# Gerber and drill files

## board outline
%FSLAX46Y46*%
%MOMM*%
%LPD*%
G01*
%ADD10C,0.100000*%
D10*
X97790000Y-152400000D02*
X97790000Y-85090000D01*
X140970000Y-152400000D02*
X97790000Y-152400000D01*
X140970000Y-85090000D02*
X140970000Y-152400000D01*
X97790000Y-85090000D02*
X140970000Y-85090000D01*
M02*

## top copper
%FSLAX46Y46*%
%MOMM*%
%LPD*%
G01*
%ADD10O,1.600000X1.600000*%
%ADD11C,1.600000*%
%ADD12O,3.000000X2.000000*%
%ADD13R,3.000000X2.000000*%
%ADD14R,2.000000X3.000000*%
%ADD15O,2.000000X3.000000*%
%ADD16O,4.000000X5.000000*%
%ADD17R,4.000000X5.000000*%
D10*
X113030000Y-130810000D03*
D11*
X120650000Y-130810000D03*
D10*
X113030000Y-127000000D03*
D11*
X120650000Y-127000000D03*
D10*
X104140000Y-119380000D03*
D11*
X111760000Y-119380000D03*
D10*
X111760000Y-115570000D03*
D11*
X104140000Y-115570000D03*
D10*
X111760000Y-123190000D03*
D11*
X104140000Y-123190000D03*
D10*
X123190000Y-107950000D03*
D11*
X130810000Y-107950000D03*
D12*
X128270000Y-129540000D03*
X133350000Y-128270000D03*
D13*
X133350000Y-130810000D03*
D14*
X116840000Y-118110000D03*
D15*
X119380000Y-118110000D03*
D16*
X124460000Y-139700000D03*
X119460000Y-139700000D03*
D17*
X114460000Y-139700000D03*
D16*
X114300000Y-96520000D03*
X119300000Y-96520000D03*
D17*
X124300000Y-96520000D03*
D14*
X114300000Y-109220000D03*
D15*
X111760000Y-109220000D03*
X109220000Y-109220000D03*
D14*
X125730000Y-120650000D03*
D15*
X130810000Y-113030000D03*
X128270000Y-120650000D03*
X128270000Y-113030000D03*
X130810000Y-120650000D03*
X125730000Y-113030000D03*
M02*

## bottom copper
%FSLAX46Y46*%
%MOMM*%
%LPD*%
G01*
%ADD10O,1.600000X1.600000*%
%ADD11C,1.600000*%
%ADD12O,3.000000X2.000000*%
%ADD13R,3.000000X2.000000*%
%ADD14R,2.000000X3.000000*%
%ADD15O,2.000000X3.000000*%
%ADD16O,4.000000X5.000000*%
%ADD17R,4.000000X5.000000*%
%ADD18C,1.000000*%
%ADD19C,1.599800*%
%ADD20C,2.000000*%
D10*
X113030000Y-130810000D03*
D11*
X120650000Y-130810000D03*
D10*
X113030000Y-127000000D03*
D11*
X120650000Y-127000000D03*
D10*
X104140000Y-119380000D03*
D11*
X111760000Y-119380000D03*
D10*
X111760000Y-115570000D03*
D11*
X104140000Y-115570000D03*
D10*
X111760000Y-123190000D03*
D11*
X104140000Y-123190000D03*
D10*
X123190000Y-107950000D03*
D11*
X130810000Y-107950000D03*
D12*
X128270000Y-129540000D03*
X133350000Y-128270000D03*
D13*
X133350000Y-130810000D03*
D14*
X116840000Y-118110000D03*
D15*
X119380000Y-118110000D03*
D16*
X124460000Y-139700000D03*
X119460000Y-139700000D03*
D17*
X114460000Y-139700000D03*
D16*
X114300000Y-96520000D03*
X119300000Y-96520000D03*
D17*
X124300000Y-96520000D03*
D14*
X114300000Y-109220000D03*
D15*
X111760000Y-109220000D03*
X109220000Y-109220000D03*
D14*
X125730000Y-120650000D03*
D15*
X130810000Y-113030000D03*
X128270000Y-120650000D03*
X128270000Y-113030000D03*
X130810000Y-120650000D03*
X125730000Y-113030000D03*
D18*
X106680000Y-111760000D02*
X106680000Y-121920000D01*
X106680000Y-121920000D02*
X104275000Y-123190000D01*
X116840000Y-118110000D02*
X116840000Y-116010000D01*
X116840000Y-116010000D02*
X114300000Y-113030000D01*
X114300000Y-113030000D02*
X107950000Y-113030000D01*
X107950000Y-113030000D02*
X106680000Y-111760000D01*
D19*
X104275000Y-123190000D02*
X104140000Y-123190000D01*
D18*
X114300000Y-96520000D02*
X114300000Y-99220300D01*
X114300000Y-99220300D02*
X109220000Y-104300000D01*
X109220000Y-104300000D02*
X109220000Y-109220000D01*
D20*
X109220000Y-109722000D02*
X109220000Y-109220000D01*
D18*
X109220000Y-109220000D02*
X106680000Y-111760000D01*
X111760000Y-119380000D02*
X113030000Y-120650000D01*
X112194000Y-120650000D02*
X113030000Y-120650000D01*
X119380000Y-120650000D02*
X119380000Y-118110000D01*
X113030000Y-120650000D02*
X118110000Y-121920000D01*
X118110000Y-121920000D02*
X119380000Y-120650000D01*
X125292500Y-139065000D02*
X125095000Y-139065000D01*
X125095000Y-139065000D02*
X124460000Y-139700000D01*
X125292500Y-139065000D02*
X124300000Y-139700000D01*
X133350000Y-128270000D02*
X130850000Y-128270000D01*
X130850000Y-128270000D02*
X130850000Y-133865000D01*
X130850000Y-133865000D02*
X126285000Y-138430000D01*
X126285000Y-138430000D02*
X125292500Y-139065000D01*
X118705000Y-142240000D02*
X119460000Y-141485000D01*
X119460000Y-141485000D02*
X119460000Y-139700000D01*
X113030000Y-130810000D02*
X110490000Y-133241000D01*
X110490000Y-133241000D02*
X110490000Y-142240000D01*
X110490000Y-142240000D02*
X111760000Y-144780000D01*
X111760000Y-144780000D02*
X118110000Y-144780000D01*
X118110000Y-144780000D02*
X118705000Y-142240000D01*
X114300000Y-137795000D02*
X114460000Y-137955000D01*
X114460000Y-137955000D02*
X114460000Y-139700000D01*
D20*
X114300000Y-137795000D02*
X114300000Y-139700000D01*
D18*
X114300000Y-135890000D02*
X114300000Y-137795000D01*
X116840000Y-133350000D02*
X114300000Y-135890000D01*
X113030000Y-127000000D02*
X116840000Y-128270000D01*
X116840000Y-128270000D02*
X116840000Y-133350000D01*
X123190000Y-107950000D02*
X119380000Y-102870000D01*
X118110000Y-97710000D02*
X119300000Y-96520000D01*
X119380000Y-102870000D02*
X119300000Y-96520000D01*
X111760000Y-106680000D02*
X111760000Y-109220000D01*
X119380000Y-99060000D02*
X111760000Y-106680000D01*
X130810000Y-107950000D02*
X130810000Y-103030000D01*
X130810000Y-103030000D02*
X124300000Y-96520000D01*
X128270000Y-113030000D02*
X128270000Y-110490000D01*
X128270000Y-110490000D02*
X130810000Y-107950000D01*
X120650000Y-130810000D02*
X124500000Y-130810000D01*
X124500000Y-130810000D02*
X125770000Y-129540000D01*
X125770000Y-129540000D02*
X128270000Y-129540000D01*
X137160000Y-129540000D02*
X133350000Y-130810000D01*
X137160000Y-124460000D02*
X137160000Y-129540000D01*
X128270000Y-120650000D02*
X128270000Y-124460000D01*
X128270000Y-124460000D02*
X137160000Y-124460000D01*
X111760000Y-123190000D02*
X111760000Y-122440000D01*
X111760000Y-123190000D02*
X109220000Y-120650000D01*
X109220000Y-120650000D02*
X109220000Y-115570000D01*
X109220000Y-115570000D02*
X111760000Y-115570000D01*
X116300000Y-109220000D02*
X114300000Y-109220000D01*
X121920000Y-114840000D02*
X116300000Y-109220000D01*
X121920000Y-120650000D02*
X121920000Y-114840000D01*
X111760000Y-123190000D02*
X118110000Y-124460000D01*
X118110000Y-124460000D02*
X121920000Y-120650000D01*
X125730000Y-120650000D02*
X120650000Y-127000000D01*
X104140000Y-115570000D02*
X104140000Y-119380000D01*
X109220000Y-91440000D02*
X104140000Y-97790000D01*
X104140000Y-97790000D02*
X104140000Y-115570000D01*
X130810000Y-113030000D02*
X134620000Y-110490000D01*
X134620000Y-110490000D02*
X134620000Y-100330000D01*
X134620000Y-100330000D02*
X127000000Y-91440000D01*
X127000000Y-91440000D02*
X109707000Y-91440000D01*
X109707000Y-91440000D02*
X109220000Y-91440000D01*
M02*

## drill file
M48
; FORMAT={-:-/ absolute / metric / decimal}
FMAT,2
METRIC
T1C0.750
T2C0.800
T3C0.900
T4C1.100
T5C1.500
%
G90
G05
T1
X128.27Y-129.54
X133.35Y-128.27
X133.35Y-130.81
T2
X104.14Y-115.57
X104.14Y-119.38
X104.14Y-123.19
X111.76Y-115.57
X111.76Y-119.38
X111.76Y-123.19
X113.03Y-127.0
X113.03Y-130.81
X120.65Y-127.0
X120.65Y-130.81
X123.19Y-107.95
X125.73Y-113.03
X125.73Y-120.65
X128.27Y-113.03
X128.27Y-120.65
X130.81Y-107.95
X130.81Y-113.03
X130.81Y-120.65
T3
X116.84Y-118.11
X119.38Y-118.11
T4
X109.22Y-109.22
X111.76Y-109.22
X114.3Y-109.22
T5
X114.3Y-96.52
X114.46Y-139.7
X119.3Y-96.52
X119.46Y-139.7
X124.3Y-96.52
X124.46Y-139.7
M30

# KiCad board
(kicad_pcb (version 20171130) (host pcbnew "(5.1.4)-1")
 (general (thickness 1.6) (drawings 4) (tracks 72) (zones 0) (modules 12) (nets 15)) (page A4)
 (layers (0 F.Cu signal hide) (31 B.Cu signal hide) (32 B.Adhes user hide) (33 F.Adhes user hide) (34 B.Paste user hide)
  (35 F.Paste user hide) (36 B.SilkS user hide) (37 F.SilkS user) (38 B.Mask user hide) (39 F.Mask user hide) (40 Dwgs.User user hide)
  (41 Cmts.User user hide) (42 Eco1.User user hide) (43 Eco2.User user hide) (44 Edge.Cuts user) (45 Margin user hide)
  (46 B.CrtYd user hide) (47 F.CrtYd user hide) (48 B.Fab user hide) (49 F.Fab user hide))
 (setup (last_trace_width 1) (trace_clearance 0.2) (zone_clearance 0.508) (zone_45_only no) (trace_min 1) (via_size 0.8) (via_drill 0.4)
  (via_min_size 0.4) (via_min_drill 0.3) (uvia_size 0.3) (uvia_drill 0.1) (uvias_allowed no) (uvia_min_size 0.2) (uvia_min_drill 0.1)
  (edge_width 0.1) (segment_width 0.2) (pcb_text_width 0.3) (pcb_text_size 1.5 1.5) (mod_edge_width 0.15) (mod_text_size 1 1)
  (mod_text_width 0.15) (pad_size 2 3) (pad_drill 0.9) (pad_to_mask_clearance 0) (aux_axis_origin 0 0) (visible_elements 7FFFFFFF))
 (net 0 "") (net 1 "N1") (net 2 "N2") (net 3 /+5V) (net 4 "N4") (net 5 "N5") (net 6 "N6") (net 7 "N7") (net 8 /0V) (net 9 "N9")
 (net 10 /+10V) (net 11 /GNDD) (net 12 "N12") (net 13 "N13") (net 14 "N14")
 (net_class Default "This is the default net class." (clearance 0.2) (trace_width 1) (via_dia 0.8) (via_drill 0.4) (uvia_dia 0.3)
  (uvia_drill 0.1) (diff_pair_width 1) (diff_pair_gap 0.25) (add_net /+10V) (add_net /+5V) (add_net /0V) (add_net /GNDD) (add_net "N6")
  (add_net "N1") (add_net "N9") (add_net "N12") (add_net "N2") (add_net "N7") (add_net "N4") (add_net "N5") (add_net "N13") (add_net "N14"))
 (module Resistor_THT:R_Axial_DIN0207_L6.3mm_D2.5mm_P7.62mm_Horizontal (layer F.Cu) (at 120.65 130.81 180)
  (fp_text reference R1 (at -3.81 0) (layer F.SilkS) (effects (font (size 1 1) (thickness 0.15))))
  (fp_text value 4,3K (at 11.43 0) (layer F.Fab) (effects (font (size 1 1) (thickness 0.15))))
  (pad 2 thru_hole oval (at 7.62 0 180) (size 1.6 1.6) (drill 0.8) (layers *.Cu *.Mask) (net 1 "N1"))
  (pad 1 thru_hole circle (at 0 0 180) (size 1.6 1.6) (drill 0.8) (layers *.Cu *.Mask) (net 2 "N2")))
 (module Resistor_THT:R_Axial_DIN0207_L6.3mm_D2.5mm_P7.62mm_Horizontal (layer F.Cu) (at 120.65 127 180)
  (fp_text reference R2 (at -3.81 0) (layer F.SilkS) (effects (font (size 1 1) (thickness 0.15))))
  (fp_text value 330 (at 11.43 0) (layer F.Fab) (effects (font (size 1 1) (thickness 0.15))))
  (pad 2 thru_hole oval (at 7.62 0 180) (size 1.6 1.6) (drill 0.8) (layers *.Cu *.Mask) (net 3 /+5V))
  (pad 1 thru_hole circle (at 0 0 180) (size 1.6 1.6) (drill 0.8) (layers *.Cu *.Mask) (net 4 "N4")))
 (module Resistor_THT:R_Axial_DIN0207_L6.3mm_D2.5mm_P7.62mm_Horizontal (layer F.Cu) (at 111.76 119.38 180)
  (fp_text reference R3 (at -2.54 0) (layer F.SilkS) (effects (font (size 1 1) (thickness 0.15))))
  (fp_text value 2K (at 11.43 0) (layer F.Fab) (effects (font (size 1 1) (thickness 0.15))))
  (pad 2 thru_hole oval (at 7.62 0 180) (size 1.6 1.6) (drill 0.8) (layers *.Cu *.Mask) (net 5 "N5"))
  (pad 1 thru_hole circle (at 0 0 180) (size 1.6 1.6) (drill 0.8) (layers *.Cu *.Mask) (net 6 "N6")))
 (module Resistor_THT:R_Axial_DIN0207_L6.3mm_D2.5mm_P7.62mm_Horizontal (layer F.Cu) (at 104.14 115.57)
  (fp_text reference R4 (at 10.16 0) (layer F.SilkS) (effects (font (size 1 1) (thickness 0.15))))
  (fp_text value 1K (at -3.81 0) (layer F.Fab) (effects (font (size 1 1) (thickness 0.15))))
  (pad 2 thru_hole oval (at 7.62 0) (size 1.6 1.6) (drill 0.8) (layers *.Cu *.Mask) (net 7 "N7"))
  (pad 1 thru_hole circle (at 0 0) (size 1.6 1.6) (drill 0.8) (layers *.Cu *.Mask) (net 5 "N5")))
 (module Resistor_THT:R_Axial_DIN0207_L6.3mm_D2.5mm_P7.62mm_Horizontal (layer F.Cu) (at 104.14 123.19)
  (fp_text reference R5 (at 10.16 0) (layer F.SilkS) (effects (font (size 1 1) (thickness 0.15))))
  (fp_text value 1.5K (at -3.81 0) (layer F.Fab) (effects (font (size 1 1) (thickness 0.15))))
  (pad 2 thru_hole oval (at 7.62 0) (size 1.6 1.6) (drill 0.8) (layers *.Cu *.Mask) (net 7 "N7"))
  (pad 1 thru_hole circle (at 0 0) (size 1.6 1.6) (drill 0.8) (layers *.Cu *.Mask) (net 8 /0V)))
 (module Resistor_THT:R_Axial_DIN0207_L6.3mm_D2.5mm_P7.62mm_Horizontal (layer F.Cu) (at 130.81 107.95 180)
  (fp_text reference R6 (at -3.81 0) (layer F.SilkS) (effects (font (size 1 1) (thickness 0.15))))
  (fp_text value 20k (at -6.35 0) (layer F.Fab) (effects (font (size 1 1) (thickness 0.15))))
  (pad 2 thru_hole oval (at 7.62 0 180) (size 1.6 1.6) (drill 0.8) (layers *.Cu *.Mask) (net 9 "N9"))
  (pad 1 thru_hole circle (at 0 0 180) (size 1.6 1.6) (drill 0.8) (layers *.Cu *.Mask) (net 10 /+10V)))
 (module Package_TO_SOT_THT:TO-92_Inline (layer F.Cu) (at 133.35 130.81 90)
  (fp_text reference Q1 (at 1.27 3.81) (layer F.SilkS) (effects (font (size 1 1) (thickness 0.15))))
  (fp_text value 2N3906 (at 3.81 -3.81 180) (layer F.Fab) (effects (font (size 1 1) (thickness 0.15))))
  (pad 2 thru_hole oval (at 1.27 -5.08 90) (size 2 3) (drill 0.75) (layers *.Cu *.Mask) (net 2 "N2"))
  (pad 3 thru_hole oval (at 2.54 0 90) (size 2 3) (drill 0.75) (layers *.Cu *.Mask) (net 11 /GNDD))
  (pad 1 thru_hole rect (at 0 0 90) (size 2 3) (drill 0.75) (layers *.Cu *.Mask) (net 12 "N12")))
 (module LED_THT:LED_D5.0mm (layer F.Cu) (at 116.84 118.11)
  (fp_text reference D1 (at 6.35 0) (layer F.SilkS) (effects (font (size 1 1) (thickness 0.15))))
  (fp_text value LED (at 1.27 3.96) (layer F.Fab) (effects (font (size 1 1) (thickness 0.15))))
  (pad 1 thru_hole rect (at 0 0) (size 2 3) (drill 0.9) (layers *.Cu *.Mask) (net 8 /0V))
  (pad 2 thru_hole oval (at 2.54 0) (size 2 3) (drill 0.9) (layers *.Cu *.Mask) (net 6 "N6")))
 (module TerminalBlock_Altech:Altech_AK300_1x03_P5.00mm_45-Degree (layer F.Cu) (at 114.46 139.7)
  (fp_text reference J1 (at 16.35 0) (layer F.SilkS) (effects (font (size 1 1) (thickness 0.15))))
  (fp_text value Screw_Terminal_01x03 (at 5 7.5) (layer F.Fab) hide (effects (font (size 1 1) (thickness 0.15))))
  (pad 3 thru_hole oval (at 10 0) (size 4 5) (drill 1.5) (layers *.Cu *.Mask) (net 11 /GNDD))
  (pad 2 thru_hole oval (at 5 0) (size 4 5) (drill 1.5) (layers *.Cu *.Mask) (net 1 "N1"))
  (pad 1 thru_hole rect (at 0 0) (size 4 5) (drill 1.5) (layers *.Cu *.Mask) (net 3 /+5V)))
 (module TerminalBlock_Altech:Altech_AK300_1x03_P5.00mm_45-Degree (layer F.Cu) (at 114.3 96.52)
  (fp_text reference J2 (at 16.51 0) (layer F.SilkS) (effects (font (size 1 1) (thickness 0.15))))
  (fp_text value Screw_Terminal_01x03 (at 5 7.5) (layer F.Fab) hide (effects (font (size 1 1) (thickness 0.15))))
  (pad 1 thru_hole oval (at 0 0) (size 4 5) (drill 1.5) (layers *.Cu *.Mask) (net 8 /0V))
  (pad 2 thru_hole oval (at 5 0) (size 4 5) (drill 1.5) (layers *.Cu *.Mask) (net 9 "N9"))
  (pad 3 thru_hole rect (at 10 0) (size 4 5) (drill 1.5) (layers *.Cu *.Mask) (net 10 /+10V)))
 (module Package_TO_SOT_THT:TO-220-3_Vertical (layer F.Cu) (at 114.3 109.22 180)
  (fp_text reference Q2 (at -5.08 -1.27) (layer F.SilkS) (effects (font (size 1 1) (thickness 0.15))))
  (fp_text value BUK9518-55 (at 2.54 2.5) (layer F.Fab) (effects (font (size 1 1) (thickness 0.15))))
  (pad 1 thru_hole rect (at 0 0 180) (size 2 3) (drill 1.1) (layers *.Cu *.Mask) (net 7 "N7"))
  (pad 2 thru_hole oval (at 2.54 0 180) (size 2 3) (drill 1.1) (layers *.Cu *.Mask) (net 9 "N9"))
  (pad 3 thru_hole oval (at 5.08 0 180) (size 2 3) (drill 1.1) (layers *.Cu *.Mask) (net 8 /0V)))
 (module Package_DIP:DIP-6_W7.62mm (layer F.Cu) (at 125.73 120.65 90)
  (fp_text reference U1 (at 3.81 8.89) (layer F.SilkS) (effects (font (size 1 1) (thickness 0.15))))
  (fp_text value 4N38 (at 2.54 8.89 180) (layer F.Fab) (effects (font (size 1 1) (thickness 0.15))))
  (pad 1 thru_hole rect (at 0 0 90) (size 3 2) (drill 0.8) (layers *.Cu *.Mask) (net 4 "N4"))
  (pad 4 thru_hole oval (at 7.62 5.08 90) (size 3 2) (drill 0.8) (layers *.Cu *.Mask) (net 5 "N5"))
  (pad 2 thru_hole oval (at 0 2.54 90) (size 3 2) (drill 0.8) (layers *.Cu *.Mask) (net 12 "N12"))
  (pad 5 thru_hole oval (at 7.62 2.54 90) (size 3 2) (drill 0.8) (layers *.Cu *.Mask) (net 10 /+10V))
  (pad 3 thru_hole oval (at 0 5.08 90) (size 3 2) (drill 0.8) (layers *.Cu *.Mask) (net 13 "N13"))
  (pad 6 thru_hole oval (at 7.62 0 90) (size 3 2) (drill 0.8) (layers *.Cu *.Mask) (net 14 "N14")))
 (gr_line (start 97.79 152.4) (end 97.79 85.09) (layer Edge.Cuts) (width 0.1))
 (gr_line (start 140.97 152.4) (end 97.79 152.4) (layer Edge.Cuts) (width 0.1))
 (gr_line (start 140.97 85.09) (end 140.97 152.4) (layer Edge.Cuts) (width 0.1))
 (gr_line (start 97.79 85.09) (end 140.97 85.09) (layer Edge.Cuts) (width 0.1))
 (segment (start 106.68 111.76) (end 106.68 121.92) (width 1) (layer B.Cu) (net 8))
 (segment (start 106.68 121.92) (end 104.275 123.19) (width 1) (layer B.Cu) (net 8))
 (segment (start 116.84 118.11) (end 116.84 116.01) (width 1) (layer B.Cu) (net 8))
 (segment (start 116.84 116.01) (end 114.3 113.03) (width 1) (layer B.Cu) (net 8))
 (segment (start 114.3 113.03) (end 107.95 113.03) (width 1) (layer B.Cu) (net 8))
 (segment (start 107.95 113.03) (end 106.68 111.76) (width 1) (layer B.Cu) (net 8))
 (segment (start 104.275 123.19) (end 104.14 123.19) (width 1.5998) (layer B.Cu) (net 8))
 (segment (start 114.3 96.52) (end 114.3 99.2203) (width 1) (layer B.Cu) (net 8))
 (segment (start 114.3 99.2203) (end 109.22 104.3) (width 1) (layer B.Cu) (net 8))
 (segment (start 109.22 104.3) (end 109.22 109.22) (width 1) (layer B.Cu) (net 8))
 (segment (start 109.22 109.722) (end 109.22 109.22) (width 2) (layer B.Cu) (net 8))
 (segment (start 109.22 109.22) (end 106.68 111.76) (width 1) (layer B.Cu) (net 8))
 (segment (start 111.76 119.38) (end 113.03 120.65) (width 1) (layer B.Cu) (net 6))
 (segment (start 112.194 120.65) (end 113.03 120.65) (width 1) (layer B.Cu) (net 6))
 (segment (start 119.38 120.65) (end 119.38 118.11) (width 1) (layer B.Cu) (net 6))
 (segment (start 113.03 120.65) (end 118.11 121.92) (width 1) (layer B.Cu) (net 6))
 (segment (start 118.11 121.92) (end 119.38 120.65) (width 1) (layer B.Cu) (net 6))
 (segment (start 125.2925 139.065) (end 125.095 139.065) (width 1) (layer B.Cu) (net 11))
 (segment (start 125.095 139.065) (end 124.46 139.7) (width 1) (layer B.Cu) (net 11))
 (segment (start 125.2925 139.065) (end 124.3 139.7) (width 1) (layer B.Cu) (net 11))
 (segment (start 133.35 128.27) (end 130.85 128.27) (width 1) (layer B.Cu) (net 11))
 (segment (start 130.85 128.27) (end 130.85 133.865) (width 1) (layer B.Cu) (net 11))
 (segment (start 130.85 133.865) (end 126.285 138.43) (width 1) (layer B.Cu) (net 11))
 (segment (start 126.285 138.43) (end 125.2925 139.065) (width 1) (layer B.Cu) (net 11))
 (segment (start 118.705 142.24) (end 119.46 141.485) (width 1) (layer B.Cu) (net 1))
 (segment (start 119.46 141.485) (end 119.46 139.7) (width 1) (layer B.Cu) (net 1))
 (segment (start 113.03 130.81) (end 110.49 133.241) (width 1) (layer B.Cu) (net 1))
 (segment (start 110.49 133.241) (end 110.49 142.24) (width 1) (layer B.Cu) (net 1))
 (segment (start 110.49 142.24) (end 111.76 144.78) (width 1) (layer B.Cu) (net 1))
 (segment (start 111.76 144.78) (end 118.11 144.78) (width 1) (layer B.Cu) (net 1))
 (segment (start 118.11 144.78) (end 118.705 142.24) (width 1) (layer B.Cu) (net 1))
 (segment (start 114.3 137.795) (end 114.46 137.955) (width 1) (layer B.Cu) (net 3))
 (segment (start 114.46 137.955) (end 114.46 139.7) (width 1) (layer B.Cu) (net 3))
 (segment (start 114.3 137.795) (end 114.3 139.7) (width 2) (layer B.Cu) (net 3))
 (segment (start 114.3 135.89) (end 114.3 137.795) (width 1) (layer B.Cu) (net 3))
 (segment (start 116.84 133.35) (end 114.3 135.89) (width 1) (layer B.Cu) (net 3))
 (segment (start 113.03 127) (end 116.84 128.27) (width 1) (layer B.Cu) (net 3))
 (segment (start 116.84 128.27) (end 116.84 133.35) (width 1) (layer B.Cu) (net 3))
 (segment (start 123.19 107.95) (end 119.38 102.87) (width 1) (layer B.Cu) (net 9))
 (segment (start 118.11 97.71) (end 119.3 96.52) (width 1) (layer B.Cu) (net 9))
 (segment (start 119.38 102.87) (end 119.3 96.52) (width 1) (layer B.Cu) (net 9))
 (segment (start 111.76 106.68) (end 111.76 109.22) (width 1) (layer B.Cu) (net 9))
 (segment (start 119.38 99.06) (end 111.76 106.68) (width 1) (layer B.Cu) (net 9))
 (segment (start 130.81 107.95) (end 130.81 103.03) (width 1) (layer B.Cu) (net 10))
 (segment (start 130.81 103.03) (end 124.3 96.52) (width 1) (layer B.Cu) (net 10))
 (segment (start 128.27 113.03) (end 128.27 110.49) (width 1) (layer B.Cu) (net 10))
 (segment (start 128.27 110.49) (end 130.81 107.95) (width 1) (layer B.Cu) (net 10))
 (segment (start 120.65 130.81) (end 124.5 130.81) (width 1) (layer B.Cu) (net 2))
 (segment (start 124.5 130.81) (end 125.77 129.54) (width 1) (layer B.Cu) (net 2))
 (segment (start 125.77 129.54) (end 128.27 129.54) (width 1) (layer B.Cu) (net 2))
 (segment (start 137.16 129.54) (end 133.35 130.81) (width 1) (layer B.Cu) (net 12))
 (segment (start 137.16 124.46) (end 137.16 129.54) (width 1) (layer B.Cu) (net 12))
 (segment (start 128.27 120.65) (end 128.27 124.46) (width 1) (layer B.Cu) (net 12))
 (segment (start 128.27 124.46) (end 137.16 124.46) (width 1) (layer B.Cu) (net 12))
 (segment (start 111.76 123.19) (end 111.76 122.44) (width 1) (layer B.Cu) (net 7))
 (segment (start 111.76 123.19) (end 109.22 120.65) (width 1) (layer B.Cu) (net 7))
 (segment (start 109.22 120.65) (end 109.22 115.57) (width 1) (layer B.Cu) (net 7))
 (segment (start 109.22 115.57) (end 111.76 115.57) (width 1) (layer B.Cu) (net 7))
 (segment (start 116.3 109.22) (end 114.3 109.22) (width 1) (layer B.Cu) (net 7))
 (segment (start 121.92 114.84) (end 116.3 109.22) (width 1) (layer B.Cu) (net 7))
 (segment (start 121.92 120.65) (end 121.92 114.84) (width 1) (layer B.Cu) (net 7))
 (segment (start 111.76 123.19) (end 118.11 124.46) (width 1) (layer B.Cu) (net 7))
 (segment (start 118.11 124.46) (end 121.92 120.65) (width 1) (layer B.Cu) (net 7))
 (segment (start 125.73 120.65) (end 120.65 127) (width 1) (layer B.Cu) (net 4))
 (segment (start 104.14 115.57) (end 104.14 119.38) (width 1) (layer B.Cu) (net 5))
 (segment (start 109.22 91.44) (end 104.14 97.79) (width 1) (layer B.Cu) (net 5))
 (segment (start 104.14 97.79) (end 104.14 115.57) (width 1) (layer B.Cu) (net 5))
 (segment (start 130.81 113.03) (end 134.62 110.49) (width 1) (layer B.Cu) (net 5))
 (segment (start 134.62 110.49) (end 134.62 100.33) (width 1) (layer B.Cu) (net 5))
 (segment (start 134.62 100.33) (end 127 91.44) (width 1) (layer B.Cu) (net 5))
 (segment (start 127 91.44) (end 109.707 91.44) (width 1) (layer B.Cu) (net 5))
 (segment (start 109.707 91.44) (end 109.22 91.44) (width 1) (layer B.Cu) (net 5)))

